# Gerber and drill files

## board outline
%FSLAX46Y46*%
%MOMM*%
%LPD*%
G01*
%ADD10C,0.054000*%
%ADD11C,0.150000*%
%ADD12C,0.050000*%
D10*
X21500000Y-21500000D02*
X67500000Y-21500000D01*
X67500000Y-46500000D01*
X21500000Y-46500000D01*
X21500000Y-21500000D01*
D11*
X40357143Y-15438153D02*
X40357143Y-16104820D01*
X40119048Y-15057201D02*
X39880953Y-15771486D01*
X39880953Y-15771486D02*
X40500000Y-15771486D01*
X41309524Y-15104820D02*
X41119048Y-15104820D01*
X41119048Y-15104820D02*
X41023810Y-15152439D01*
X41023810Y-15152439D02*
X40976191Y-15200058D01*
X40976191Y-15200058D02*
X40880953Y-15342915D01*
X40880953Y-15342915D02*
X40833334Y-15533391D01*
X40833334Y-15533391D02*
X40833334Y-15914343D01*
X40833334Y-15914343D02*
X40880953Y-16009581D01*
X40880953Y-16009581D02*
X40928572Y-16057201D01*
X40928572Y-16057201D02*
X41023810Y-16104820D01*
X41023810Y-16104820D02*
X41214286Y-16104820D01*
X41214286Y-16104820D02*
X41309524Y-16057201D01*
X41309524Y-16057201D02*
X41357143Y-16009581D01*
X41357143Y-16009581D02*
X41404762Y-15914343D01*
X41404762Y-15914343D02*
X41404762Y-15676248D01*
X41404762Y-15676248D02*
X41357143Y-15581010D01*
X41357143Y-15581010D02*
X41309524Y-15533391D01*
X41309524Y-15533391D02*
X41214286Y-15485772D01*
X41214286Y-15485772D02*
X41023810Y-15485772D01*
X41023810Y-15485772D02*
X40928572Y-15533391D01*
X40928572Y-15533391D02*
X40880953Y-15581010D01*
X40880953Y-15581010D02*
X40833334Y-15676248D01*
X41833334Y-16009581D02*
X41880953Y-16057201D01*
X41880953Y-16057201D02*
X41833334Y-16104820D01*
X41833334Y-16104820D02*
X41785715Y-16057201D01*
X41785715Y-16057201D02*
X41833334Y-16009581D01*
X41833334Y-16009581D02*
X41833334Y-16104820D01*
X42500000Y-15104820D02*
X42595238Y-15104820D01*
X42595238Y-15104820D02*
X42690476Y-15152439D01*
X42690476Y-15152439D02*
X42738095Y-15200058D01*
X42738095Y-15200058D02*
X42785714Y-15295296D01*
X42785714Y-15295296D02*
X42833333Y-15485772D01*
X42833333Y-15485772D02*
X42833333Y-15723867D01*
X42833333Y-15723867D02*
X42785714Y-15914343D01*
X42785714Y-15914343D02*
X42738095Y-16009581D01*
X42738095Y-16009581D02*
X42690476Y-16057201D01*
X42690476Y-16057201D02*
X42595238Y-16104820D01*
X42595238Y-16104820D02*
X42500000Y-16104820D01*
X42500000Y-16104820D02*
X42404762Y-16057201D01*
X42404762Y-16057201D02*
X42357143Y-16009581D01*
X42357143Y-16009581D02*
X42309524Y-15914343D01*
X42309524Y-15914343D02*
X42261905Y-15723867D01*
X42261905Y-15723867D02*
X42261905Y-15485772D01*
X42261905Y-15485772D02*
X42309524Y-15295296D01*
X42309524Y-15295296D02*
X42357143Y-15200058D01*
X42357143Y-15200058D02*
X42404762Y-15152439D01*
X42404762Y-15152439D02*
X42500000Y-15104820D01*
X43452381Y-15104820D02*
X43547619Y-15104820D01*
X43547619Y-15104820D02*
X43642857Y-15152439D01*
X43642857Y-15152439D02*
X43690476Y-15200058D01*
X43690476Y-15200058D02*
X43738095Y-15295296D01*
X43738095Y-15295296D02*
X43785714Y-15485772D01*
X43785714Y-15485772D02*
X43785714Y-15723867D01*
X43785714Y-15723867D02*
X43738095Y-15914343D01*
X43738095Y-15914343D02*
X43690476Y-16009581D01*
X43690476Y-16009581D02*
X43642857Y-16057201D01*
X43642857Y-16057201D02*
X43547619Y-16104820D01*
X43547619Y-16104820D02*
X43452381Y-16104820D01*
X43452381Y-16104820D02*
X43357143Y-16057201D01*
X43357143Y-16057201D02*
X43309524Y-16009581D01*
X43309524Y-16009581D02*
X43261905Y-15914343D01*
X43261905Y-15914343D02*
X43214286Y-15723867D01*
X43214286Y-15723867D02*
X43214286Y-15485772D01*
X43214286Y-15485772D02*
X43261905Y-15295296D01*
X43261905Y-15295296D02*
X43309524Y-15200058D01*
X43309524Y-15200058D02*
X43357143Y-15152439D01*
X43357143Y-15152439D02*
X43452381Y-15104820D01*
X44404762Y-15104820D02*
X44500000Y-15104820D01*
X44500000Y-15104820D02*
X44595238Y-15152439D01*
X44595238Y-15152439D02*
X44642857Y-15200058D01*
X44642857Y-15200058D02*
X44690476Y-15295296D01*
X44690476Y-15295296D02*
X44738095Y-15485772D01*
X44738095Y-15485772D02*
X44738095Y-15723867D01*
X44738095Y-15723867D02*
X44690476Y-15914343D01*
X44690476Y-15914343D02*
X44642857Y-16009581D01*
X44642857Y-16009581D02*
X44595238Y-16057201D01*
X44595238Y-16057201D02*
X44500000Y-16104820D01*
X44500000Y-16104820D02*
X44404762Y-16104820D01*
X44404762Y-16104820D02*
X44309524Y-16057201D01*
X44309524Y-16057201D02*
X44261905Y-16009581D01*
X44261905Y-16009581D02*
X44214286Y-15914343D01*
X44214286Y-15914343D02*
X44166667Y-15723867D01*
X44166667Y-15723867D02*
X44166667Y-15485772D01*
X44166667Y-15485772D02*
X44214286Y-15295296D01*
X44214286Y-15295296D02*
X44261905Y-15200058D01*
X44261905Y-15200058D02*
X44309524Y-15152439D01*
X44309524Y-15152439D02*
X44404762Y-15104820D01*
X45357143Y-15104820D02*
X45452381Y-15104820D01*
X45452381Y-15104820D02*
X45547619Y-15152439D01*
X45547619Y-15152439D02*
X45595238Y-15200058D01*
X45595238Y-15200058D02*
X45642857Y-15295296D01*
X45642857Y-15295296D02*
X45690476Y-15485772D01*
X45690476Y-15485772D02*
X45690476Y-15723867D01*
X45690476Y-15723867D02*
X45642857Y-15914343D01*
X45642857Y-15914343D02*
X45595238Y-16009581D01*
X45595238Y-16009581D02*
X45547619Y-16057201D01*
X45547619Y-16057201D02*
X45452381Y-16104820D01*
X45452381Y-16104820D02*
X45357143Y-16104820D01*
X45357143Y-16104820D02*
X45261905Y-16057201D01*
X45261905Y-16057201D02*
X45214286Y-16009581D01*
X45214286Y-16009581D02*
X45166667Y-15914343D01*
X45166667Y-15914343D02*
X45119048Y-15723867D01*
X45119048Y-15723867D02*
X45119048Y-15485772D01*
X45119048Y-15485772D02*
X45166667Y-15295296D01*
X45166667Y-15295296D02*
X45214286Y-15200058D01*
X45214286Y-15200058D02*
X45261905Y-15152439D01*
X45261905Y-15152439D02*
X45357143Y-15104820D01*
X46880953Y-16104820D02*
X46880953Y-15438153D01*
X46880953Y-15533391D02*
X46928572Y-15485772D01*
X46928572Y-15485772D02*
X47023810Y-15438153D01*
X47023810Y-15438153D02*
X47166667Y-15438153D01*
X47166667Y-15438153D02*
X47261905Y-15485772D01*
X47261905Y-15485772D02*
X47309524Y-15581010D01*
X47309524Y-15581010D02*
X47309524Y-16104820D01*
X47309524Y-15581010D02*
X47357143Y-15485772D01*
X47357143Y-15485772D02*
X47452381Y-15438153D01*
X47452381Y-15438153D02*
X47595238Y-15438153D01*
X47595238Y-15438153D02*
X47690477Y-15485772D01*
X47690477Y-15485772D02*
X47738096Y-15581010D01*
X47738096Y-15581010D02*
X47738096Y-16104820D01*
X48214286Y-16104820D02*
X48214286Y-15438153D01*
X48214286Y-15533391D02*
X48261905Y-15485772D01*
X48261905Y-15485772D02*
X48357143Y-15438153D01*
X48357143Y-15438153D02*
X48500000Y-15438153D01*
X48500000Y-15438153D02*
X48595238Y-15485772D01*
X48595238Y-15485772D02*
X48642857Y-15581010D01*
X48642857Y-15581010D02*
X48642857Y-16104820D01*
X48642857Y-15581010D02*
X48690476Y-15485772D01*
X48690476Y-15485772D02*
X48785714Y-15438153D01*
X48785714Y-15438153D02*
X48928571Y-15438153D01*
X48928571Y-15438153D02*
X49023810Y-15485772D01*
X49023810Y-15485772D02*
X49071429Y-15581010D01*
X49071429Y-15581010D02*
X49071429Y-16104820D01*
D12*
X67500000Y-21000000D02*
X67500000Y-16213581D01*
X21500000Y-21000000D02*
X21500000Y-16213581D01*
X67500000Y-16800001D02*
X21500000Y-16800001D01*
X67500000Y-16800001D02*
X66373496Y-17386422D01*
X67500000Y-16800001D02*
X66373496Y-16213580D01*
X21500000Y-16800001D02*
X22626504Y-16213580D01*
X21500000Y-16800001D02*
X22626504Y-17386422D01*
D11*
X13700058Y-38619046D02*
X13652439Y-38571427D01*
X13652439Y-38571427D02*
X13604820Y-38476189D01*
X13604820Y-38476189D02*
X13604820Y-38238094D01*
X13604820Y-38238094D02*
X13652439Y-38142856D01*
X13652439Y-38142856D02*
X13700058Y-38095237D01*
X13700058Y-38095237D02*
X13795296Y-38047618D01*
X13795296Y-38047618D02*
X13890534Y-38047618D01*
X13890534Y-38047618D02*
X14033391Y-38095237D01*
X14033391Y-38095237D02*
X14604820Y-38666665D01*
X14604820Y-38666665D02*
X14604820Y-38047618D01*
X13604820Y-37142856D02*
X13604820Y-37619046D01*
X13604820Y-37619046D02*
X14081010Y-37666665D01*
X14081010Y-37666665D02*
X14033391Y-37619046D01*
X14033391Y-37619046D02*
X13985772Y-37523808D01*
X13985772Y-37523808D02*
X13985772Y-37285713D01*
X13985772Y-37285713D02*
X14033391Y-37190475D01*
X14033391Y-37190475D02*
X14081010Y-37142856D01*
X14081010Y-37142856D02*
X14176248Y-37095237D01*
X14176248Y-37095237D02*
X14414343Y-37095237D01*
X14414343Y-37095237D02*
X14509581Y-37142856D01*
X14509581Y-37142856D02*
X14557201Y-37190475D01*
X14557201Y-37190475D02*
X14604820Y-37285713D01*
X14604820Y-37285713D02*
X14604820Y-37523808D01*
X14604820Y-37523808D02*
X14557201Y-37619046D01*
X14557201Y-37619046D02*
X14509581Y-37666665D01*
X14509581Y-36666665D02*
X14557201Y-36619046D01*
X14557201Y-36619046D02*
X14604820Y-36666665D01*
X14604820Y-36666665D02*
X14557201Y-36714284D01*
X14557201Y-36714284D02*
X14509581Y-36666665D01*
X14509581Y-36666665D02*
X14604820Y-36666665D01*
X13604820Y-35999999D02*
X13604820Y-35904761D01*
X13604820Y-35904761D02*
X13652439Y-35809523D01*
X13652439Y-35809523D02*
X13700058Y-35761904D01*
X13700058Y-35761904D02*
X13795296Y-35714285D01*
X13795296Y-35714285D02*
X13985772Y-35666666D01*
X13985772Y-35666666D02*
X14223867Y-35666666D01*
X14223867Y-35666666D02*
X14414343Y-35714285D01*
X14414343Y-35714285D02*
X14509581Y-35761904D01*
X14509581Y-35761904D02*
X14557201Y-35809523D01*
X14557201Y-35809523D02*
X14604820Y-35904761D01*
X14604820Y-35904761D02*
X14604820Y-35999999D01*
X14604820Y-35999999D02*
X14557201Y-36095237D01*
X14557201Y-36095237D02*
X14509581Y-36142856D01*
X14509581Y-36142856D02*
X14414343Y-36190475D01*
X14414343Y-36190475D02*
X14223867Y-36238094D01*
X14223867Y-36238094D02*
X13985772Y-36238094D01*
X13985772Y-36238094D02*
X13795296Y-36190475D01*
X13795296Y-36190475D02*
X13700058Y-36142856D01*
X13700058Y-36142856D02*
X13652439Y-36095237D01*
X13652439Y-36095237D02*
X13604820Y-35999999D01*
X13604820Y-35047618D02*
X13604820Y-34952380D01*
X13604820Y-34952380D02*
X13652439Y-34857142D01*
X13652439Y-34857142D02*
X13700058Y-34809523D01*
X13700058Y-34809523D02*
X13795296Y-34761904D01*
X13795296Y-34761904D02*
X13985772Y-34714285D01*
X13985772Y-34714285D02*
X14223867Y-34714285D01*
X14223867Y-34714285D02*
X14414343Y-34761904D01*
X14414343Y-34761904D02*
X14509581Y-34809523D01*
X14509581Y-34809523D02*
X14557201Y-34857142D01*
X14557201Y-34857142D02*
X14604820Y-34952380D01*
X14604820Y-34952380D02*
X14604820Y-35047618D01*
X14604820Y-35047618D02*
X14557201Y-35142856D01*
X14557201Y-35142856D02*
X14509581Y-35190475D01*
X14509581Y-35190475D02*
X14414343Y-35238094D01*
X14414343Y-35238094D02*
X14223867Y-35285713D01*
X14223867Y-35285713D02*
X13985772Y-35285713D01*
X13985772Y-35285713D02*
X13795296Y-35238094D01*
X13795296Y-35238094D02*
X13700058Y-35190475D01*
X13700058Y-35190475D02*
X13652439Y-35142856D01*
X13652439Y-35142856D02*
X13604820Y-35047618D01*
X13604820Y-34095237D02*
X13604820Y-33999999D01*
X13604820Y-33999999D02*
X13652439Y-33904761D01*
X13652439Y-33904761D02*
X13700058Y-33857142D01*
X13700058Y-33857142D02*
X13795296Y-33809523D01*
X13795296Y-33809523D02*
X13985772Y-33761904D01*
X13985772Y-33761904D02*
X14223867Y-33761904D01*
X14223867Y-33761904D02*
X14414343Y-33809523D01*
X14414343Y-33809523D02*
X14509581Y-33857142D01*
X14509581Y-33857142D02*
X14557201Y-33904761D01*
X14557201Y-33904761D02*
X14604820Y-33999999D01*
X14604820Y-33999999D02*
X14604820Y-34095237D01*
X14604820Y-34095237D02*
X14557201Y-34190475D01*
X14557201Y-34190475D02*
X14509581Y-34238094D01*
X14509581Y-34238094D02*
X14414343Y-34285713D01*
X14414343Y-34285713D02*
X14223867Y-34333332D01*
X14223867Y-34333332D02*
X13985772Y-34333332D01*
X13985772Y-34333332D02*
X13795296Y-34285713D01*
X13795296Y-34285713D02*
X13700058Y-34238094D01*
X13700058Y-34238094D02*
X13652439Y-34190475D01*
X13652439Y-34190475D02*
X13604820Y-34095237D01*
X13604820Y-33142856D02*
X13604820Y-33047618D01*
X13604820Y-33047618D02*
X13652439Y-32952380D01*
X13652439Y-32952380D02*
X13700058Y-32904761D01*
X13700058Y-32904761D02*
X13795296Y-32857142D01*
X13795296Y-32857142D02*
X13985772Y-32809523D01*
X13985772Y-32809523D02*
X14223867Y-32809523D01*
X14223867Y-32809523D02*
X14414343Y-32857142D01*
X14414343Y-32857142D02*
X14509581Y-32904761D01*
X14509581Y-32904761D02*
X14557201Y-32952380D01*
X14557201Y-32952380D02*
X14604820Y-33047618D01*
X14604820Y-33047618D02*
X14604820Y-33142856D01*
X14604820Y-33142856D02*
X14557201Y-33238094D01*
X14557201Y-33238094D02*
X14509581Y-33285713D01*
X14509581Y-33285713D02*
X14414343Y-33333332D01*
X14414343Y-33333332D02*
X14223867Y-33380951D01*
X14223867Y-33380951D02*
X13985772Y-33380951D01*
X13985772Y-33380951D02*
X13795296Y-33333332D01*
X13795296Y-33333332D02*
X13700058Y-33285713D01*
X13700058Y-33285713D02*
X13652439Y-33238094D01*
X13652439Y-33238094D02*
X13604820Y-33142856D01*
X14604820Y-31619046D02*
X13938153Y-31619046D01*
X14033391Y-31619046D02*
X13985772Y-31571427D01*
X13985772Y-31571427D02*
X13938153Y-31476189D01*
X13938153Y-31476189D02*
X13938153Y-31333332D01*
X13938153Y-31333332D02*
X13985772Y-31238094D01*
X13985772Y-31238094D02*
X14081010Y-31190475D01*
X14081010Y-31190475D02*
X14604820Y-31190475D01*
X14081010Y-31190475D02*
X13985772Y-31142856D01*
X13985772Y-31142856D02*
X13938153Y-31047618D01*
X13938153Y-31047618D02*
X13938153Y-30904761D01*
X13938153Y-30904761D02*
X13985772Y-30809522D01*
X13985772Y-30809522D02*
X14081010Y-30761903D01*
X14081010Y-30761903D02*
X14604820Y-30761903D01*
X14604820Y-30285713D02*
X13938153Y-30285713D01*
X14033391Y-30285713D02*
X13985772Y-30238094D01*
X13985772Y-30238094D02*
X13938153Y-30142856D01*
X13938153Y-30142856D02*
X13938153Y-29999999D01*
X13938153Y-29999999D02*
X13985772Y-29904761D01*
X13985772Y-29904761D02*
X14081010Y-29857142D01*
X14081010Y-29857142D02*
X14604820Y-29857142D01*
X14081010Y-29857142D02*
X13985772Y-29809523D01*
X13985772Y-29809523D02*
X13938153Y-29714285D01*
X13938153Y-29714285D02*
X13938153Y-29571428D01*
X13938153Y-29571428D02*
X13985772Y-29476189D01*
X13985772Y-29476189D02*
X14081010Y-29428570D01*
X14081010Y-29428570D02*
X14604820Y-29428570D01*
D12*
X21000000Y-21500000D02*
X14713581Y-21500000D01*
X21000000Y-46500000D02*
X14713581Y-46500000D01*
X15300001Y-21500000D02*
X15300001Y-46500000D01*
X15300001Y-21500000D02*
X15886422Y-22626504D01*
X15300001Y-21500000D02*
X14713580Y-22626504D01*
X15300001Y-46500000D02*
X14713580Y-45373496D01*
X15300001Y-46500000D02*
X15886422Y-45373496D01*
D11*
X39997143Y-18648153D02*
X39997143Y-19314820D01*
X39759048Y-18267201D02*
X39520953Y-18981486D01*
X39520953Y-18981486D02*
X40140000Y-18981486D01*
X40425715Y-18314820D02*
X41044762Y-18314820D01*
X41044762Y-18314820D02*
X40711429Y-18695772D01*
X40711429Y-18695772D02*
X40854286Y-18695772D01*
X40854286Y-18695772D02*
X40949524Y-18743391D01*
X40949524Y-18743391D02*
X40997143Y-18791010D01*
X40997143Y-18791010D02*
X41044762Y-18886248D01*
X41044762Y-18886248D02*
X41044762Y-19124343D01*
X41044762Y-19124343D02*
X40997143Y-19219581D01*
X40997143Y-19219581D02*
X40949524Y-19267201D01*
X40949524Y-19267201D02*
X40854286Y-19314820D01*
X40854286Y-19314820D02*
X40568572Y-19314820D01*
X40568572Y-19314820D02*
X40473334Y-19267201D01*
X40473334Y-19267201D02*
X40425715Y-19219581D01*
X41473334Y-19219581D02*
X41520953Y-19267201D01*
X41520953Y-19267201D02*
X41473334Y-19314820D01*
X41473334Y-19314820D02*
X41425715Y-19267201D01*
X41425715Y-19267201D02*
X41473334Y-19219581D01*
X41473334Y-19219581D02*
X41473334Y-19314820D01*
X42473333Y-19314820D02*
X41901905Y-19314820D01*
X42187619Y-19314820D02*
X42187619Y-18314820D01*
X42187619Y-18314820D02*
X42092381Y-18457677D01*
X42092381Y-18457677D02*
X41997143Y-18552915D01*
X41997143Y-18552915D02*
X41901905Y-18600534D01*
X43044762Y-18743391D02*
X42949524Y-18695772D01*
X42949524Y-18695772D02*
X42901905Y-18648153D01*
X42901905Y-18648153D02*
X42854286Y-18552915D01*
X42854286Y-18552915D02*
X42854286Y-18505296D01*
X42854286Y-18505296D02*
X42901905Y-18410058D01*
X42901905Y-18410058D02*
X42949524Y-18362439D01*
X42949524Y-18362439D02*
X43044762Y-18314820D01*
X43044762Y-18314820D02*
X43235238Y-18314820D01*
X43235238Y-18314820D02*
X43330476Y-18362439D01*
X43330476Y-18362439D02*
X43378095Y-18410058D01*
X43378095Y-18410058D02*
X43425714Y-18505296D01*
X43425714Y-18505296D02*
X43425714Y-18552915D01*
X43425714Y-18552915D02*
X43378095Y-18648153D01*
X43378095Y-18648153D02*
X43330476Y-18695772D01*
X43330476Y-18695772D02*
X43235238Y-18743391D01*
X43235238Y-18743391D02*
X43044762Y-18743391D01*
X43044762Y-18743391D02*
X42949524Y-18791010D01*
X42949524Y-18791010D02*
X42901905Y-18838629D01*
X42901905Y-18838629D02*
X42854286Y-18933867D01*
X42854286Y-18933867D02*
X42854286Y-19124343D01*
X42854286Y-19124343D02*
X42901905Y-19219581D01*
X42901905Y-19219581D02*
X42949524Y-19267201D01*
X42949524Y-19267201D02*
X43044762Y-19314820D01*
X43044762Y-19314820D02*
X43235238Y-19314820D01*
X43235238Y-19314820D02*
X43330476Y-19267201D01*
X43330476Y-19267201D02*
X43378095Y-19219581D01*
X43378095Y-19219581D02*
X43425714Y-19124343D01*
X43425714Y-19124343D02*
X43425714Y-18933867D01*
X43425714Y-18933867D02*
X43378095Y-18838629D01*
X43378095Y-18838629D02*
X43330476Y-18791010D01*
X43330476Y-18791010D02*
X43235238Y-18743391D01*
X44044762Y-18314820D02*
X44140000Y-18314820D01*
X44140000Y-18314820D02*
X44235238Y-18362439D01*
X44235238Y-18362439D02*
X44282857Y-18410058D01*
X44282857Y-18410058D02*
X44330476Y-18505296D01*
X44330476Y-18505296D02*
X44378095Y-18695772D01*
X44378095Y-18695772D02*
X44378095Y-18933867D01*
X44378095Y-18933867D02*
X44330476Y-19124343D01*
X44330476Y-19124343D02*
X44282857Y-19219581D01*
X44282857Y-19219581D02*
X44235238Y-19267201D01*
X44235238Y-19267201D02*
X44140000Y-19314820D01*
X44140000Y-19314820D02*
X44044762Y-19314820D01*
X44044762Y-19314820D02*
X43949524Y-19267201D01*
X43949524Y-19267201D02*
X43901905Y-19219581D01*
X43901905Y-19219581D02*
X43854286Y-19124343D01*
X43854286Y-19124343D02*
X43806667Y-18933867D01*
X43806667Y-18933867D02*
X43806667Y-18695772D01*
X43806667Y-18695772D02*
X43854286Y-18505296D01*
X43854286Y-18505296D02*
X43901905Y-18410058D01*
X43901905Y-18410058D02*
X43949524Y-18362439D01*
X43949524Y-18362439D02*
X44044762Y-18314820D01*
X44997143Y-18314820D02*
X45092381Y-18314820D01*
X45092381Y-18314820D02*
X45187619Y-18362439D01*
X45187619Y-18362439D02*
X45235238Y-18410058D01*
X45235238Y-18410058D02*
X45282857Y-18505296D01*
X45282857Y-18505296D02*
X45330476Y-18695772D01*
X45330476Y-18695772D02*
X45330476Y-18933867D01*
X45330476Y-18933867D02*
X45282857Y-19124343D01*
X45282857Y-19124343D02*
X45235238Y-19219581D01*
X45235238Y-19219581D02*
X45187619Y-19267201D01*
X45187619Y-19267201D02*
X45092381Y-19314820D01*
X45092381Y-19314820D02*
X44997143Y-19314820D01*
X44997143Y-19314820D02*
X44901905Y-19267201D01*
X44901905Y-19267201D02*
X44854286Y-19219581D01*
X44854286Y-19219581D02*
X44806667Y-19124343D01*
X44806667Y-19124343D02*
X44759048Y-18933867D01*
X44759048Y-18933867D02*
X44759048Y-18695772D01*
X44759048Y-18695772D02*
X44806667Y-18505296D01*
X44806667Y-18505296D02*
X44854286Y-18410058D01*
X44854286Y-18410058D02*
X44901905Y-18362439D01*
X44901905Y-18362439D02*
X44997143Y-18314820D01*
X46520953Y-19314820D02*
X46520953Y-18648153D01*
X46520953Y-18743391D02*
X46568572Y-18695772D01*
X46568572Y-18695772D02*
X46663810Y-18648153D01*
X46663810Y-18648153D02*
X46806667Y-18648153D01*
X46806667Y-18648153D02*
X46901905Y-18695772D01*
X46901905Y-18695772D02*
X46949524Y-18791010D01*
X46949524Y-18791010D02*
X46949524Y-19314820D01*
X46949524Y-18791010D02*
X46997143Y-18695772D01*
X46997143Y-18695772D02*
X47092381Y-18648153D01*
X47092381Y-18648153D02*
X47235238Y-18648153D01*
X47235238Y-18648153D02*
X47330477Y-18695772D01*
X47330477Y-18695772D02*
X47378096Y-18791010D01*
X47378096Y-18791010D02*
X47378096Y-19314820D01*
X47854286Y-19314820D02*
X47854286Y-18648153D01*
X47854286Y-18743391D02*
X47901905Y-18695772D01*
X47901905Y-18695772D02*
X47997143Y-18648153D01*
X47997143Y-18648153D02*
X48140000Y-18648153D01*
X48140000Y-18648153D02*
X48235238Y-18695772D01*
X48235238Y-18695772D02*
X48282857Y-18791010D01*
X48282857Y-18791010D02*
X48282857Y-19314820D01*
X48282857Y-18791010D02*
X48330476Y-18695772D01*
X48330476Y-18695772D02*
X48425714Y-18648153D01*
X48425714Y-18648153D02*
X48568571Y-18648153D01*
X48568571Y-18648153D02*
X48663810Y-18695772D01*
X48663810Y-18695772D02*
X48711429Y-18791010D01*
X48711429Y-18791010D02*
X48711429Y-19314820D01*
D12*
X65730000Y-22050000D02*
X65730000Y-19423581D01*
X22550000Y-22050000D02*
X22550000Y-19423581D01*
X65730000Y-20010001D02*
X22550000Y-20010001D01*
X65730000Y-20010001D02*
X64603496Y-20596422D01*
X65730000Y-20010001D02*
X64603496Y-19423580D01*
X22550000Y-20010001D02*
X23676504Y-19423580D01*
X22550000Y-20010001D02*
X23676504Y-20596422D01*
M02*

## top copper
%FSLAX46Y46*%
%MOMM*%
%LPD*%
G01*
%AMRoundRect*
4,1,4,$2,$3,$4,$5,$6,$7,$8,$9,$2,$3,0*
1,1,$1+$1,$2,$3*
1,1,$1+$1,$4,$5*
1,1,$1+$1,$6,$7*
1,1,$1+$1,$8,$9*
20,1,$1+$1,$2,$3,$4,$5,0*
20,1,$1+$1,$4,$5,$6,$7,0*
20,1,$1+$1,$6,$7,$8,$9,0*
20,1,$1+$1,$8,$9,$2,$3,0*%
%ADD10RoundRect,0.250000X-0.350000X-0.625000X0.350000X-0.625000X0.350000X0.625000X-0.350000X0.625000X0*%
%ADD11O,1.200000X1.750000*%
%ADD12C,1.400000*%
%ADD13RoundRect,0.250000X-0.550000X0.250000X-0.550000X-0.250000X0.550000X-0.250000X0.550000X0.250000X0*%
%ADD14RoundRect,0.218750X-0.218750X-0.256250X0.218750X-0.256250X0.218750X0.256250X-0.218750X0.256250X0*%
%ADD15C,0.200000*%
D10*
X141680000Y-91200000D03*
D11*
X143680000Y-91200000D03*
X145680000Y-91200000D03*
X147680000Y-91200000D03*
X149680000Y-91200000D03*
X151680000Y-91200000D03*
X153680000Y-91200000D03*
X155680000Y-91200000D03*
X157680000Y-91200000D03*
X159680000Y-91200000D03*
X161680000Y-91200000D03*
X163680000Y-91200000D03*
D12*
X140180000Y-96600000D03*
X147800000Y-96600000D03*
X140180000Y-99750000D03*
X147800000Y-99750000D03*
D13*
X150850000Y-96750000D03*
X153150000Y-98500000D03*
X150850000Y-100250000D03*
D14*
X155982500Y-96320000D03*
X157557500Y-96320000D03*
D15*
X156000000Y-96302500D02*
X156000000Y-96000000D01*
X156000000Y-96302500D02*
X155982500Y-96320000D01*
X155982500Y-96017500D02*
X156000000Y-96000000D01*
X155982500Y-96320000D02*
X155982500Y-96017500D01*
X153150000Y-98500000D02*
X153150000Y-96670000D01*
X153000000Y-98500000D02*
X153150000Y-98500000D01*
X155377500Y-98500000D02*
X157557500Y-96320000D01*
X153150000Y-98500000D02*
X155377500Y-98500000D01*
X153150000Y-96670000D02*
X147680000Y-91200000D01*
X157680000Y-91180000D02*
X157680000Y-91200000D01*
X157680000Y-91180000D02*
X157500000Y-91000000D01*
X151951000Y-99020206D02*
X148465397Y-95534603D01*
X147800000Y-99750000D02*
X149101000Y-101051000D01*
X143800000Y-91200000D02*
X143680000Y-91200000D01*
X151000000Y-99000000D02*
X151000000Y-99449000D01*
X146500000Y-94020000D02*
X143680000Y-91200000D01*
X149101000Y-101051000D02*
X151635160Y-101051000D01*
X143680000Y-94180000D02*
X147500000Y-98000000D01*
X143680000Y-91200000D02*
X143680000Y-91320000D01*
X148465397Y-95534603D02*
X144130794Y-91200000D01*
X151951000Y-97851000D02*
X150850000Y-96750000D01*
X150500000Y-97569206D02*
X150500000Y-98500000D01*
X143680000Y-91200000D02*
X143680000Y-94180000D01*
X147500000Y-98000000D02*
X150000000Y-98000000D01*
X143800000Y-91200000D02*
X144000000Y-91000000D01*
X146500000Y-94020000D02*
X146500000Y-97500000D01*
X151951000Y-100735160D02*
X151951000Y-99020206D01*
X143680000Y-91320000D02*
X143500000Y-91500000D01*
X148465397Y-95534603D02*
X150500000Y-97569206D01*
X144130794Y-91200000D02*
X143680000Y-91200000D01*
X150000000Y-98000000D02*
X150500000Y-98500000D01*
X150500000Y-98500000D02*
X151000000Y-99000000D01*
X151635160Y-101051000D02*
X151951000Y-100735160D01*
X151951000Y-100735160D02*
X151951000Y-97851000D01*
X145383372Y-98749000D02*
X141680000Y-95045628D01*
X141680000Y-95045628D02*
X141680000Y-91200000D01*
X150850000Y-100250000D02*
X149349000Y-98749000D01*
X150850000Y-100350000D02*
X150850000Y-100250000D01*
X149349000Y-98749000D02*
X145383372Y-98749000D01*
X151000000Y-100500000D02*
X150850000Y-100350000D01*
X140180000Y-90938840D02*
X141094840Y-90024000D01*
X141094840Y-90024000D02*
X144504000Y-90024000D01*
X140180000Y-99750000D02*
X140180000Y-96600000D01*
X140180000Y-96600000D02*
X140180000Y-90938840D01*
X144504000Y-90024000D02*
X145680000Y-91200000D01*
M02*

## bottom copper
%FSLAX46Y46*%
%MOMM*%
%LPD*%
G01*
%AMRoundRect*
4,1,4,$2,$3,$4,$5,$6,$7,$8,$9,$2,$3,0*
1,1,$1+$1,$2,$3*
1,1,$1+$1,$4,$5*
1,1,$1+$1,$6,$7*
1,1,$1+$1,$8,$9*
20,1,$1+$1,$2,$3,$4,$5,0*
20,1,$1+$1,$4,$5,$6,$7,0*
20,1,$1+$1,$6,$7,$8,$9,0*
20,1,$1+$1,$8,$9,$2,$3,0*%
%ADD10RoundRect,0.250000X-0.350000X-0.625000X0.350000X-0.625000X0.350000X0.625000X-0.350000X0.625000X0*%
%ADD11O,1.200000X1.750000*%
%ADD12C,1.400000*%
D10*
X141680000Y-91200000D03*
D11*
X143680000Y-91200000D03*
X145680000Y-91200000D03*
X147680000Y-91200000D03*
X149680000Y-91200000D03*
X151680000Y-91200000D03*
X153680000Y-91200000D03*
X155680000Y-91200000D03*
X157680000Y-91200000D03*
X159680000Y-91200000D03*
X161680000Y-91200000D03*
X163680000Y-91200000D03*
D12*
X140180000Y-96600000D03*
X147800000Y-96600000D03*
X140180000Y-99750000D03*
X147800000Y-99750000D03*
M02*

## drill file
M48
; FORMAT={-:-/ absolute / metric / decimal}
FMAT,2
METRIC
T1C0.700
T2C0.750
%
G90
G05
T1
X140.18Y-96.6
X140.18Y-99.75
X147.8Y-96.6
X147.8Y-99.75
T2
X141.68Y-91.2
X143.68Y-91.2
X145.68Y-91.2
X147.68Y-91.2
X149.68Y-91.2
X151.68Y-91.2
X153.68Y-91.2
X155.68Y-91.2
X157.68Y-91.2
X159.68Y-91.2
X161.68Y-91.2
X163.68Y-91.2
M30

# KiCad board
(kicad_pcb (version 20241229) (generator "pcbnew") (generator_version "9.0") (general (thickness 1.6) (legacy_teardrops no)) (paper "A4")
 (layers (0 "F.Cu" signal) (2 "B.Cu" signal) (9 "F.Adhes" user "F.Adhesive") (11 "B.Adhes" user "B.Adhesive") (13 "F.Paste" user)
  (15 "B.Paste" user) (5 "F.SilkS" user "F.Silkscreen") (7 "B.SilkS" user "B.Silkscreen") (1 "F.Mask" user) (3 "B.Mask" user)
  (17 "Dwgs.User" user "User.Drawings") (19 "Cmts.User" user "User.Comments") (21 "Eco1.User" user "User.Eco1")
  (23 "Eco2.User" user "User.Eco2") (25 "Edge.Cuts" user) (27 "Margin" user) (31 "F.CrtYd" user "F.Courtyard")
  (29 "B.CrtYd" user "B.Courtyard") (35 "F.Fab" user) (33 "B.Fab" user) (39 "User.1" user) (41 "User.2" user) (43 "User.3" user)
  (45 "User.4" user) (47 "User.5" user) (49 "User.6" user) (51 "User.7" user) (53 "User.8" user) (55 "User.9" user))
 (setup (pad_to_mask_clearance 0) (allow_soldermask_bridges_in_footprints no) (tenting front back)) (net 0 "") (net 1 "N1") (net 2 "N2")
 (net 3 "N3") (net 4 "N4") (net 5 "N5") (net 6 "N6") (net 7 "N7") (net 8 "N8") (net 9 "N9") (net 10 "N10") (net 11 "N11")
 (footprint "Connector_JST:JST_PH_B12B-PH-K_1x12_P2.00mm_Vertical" (layer "F.Cu") (at 141.68 91.2)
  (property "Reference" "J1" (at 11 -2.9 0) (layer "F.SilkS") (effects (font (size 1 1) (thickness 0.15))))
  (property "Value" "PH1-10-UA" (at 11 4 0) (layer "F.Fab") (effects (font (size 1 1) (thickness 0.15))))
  (pad "1" thru_hole roundrect (at 0 0) (size 1.2 1.75) (drill 0.75) (layers "*.Cu" "*.Mask") (remove_unused_layers no)
   (roundrect_rratio 0.208333) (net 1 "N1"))
  (pad "2" thru_hole oval (at 2 0) (size 1.2 1.75) (drill 0.75) (layers "*.Cu" "*.Mask") (remove_unused_layers no) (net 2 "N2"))
  (pad "3" thru_hole oval (at 4 0) (size 1.2 1.75) (drill 0.75) (layers "*.Cu" "*.Mask") (remove_unused_layers no) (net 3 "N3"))
  (pad "4" thru_hole oval (at 6 0) (size 1.2 1.75) (drill 0.75) (layers "*.Cu" "*.Mask") (remove_unused_layers no) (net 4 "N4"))
  (pad "5" thru_hole oval (at 8 0) (size 1.2 1.75) (drill 0.75) (layers "*.Cu" "*.Mask") (remove_unused_layers no) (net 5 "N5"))
  (pad "6" thru_hole oval (at 10 0) (size 1.2 1.75) (drill 0.75) (layers "*.Cu" "*.Mask") (remove_unused_layers no) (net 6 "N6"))
  (pad "7" thru_hole oval (at 12 0) (size 1.2 1.75) (drill 0.75) (layers "*.Cu" "*.Mask") (remove_unused_layers no) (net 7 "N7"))
  (pad "8" thru_hole oval (at 14 0) (size 1.2 1.75) (drill 0.75) (layers "*.Cu" "*.Mask") (remove_unused_layers no) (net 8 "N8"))
  (pad "9" thru_hole oval (at 16 0) (size 1.2 1.75) (drill 0.75) (layers "*.Cu" "*.Mask") (remove_unused_layers no) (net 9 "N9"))
  (pad "10" thru_hole oval (at 18 0) (size 1.2 1.75) (drill 0.75) (layers "*.Cu" "*.Mask") (remove_unused_layers no) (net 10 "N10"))
  (pad "11" thru_hole oval (at 20 0) (size 1.2 1.75) (drill 0.75) (layers "*.Cu" "*.Mask") (remove_unused_layers no))
  (pad "12" thru_hole oval (at 22 0) (size 1.2 1.75) (drill 0.75) (layers "*.Cu" "*.Mask") (remove_unused_layers no)))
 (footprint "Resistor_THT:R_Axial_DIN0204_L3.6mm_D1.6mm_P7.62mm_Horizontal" (layer "F.Cu") (at 140.18 96.6)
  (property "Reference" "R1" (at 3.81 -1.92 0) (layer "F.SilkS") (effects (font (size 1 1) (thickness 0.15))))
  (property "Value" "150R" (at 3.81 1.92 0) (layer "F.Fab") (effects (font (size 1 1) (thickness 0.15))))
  (pad "1" thru_hole circle (at 0 0) (size 1.4 1.4) (drill 0.7) (layers "*.Cu" "*.Mask") (remove_unused_layers no) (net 3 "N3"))
  (pad "2" thru_hole circle (at 7.62 0) (size 1.4 1.4) (drill 0.7) (layers "*.Cu" "*.Mask") (remove_unused_layers no) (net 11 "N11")))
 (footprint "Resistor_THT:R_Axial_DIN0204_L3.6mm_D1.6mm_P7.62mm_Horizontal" (layer "F.Cu") (at 140.18 99.75)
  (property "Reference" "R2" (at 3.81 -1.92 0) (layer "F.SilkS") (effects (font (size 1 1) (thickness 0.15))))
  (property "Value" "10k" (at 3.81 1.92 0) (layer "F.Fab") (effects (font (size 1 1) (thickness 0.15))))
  (pad "1" thru_hole circle (at 0 0) (size 1.4 1.4) (drill 0.7) (layers "*.Cu" "*.Mask") (remove_unused_layers no) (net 3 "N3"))
  (pad "2" thru_hole circle (at 7.62 0) (size 1.4 1.4) (drill 0.7) (layers "*.Cu" "*.Mask") (remove_unused_layers no) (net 2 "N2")))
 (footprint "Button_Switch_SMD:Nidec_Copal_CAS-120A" (layer "F.Cu") (at 152 98.5)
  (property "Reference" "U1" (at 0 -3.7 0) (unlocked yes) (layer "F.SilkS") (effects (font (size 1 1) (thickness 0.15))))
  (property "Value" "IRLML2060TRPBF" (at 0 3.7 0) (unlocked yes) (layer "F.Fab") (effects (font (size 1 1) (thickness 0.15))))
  (pad "1" smd roundrect (at -1.15 -1.75 270) (size 1 1.6) (layers "F.Cu" "F.Mask" "F.Paste") (roundrect_rratio 0.25) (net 2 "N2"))
  (pad "2" smd roundrect (at 1.15 0 270) (size 1 1.6) (layers "F.Cu" "F.Mask" "F.Paste") (roundrect_rratio 0.25) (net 4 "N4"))
  (pad "3" smd roundrect (at -1.15 1.75 270) (size 1 1.6) (layers "F.Cu" "F.Mask" "F.Paste") (roundrect_rratio 0.25) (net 1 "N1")))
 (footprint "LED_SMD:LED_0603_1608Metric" (layer "F.Cu") (at 156.77 96.32)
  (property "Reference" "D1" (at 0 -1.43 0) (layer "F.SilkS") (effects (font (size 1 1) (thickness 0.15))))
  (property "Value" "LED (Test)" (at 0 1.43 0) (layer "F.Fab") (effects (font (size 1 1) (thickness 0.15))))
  (pad "1" smd roundrect (at -0.7875 0) (size 0.875 0.95) (layers "F.Cu" "F.Mask" "F.Paste") (roundrect_rratio 0.25) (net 11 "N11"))
  (pad "2" smd roundrect (at 0.7875 0) (size 0.875 0.95) (layers "F.Cu" "F.Mask" "F.Paste") (roundrect_rratio 0.25) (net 4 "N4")))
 (gr_rect (start 21.5 21.5) (end 67.5 46.5) (stroke (width 0.054) (type default)) (fill no) (layer "Edge.Cuts"))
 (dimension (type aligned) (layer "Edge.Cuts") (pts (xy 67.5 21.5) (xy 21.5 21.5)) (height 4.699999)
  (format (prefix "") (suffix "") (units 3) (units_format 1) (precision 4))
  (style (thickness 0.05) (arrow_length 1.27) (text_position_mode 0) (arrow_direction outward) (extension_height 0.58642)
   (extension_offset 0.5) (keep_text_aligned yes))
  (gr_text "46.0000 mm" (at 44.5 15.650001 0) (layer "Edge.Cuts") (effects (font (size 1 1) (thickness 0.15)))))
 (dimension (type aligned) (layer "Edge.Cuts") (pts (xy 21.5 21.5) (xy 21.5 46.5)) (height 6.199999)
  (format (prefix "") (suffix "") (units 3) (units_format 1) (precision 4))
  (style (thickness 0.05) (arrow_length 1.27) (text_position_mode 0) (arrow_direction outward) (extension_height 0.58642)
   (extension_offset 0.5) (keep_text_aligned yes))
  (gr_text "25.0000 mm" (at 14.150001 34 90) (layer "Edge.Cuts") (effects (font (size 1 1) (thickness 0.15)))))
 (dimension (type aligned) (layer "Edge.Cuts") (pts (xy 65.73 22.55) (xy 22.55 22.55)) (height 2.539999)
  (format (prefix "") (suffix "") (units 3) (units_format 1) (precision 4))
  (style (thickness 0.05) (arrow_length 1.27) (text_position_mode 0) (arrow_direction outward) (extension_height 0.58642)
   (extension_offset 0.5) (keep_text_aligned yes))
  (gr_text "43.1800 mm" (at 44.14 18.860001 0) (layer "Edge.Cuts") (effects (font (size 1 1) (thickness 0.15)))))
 (segment (start 156 96.3025) (end 156 96) (width 0.2) (layer "F.Cu") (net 11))
 (segment (start 156 96.3025) (end 155.9825 96.32) (width 0.2) (layer "F.Cu") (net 11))
 (segment (start 155.9825 96.0175) (end 156 96) (width 0.2) (layer "F.Cu") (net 11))
 (segment (start 155.9825 96.32) (end 155.9825 96.0175) (width 0.2) (layer "F.Cu") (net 11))
 (segment (start 153.15 98.5) (end 153.15 96.67) (width 0.2) (layer "F.Cu") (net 4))
 (segment (start 153 98.5) (end 153.15 98.5) (width 0.2) (layer "F.Cu") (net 4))
 (segment (start 155.3775 98.5) (end 157.5575 96.32) (width 0.2) (layer "F.Cu") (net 4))
 (segment (start 153.15 98.5) (end 155.3775 98.5) (width 0.2) (layer "F.Cu") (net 4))
 (segment (start 153.15 96.67) (end 147.68 91.2) (width 0.2) (layer "F.Cu") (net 4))
 (segment (start 157.68 91.18) (end 157.68 91.2) (width 0.2) (layer "F.Cu") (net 9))
 (segment (start 157.68 91.18) (end 157.5 91) (width 0.2) (layer "F.Cu") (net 9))
 (segment (start 151.951 99.020206) (end 148.465397 95.534603) (width 0.2) (layer "F.Cu") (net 2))
 (segment (start 147.8 99.75) (end 149.101 101.051) (width 0.2) (layer "F.Cu") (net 2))
 (segment (start 143.8 91.2) (end 143.68 91.2) (width 0.2) (layer "F.Cu") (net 2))
 (segment (start 151 99) (end 151 99.449) (width 0.2) (layer "F.Cu") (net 2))
 (segment (start 146.5 94.02) (end 143.68 91.2) (width 0.2) (layer "F.Cu") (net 2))
 (segment (start 149.101 101.051) (end 151.63516 101.051) (width 0.2) (layer "F.Cu") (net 2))
 (segment (start 143.68 94.18) (end 147.5 98) (width 0.2) (layer "F.Cu") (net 2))
 (segment (start 143.68 91.2) (end 143.68 91.32) (width 0.2) (layer "F.Cu") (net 2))
 (segment (start 148.465397 95.534603) (end 144.130794 91.2) (width 0.2) (layer "F.Cu") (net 2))
 (segment (start 151.951 97.851) (end 150.85 96.75) (width 0.2) (layer "F.Cu") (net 2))
 (segment (start 150.5 97.569206) (end 150.5 98.5) (width 0.2) (layer "F.Cu") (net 2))
 (segment (start 143.68 91.2) (end 143.68 94.18) (width 0.2) (layer "F.Cu") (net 2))
 (segment (start 147.5 98) (end 150 98) (width 0.2) (layer "F.Cu") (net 2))
 (segment (start 143.8 91.2) (end 144 91) (width 0.2) (layer "F.Cu") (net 2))
 (segment (start 146.5 94.02) (end 146.5 97.5) (width 0.2) (layer "F.Cu") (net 2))
 (segment (start 151.951 100.73516) (end 151.951 99.020206) (width 0.2) (layer "F.Cu") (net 2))
 (segment (start 143.68 91.32) (end 143.5 91.5) (width 0.2) (layer "F.Cu") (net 2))
 (segment (start 148.465397 95.534603) (end 150.5 97.569206) (width 0.2) (layer "F.Cu") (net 2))
 (segment (start 144.130794 91.2) (end 143.68 91.2) (width 0.2) (layer "F.Cu") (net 2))
 (segment (start 150 98) (end 150.5 98.5) (width 0.2) (layer "F.Cu") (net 2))
 (segment (start 150.5 98.5) (end 151 99) (width 0.2) (layer "F.Cu") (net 2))
 (segment (start 151.63516 101.051) (end 151.951 100.73516) (width 0.2) (layer "F.Cu") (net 2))
 (segment (start 151.951 100.73516) (end 151.951 97.851) (width 0.2) (layer "F.Cu") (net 2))
 (segment (start 145.383372 98.749) (end 141.68 95.045628) (width 0.2) (layer "F.Cu") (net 1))
 (segment (start 141.68 95.045628) (end 141.68 91.2) (width 0.2) (layer "F.Cu") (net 1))
 (segment (start 150.85 100.25) (end 149.349 98.749) (width 0.2) (layer "F.Cu") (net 1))
 (segment (start 150.85 100.35) (end 150.85 100.25) (width 0.2) (layer "F.Cu") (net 1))
 (segment (start 149.349 98.749) (end 145.383372 98.749) (width 0.2) (layer "F.Cu") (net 1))
 (segment (start 151 100.5) (end 150.85 100.35) (width 0.2) (layer "F.Cu") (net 1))
 (segment (start 140.18 90.93884) (end 141.09484 90.024) (width 0.2) (layer "F.Cu") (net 3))
 (segment (start 141.09484 90.024) (end 144.504 90.024) (width 0.2) (layer "F.Cu") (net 3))
 (segment (start 140.18 99.75) (end 140.18 96.6) (width 0.2) (layer "F.Cu") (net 3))
 (segment (start 140.18 96.6) (end 140.18 90.93884) (width 0.2) (layer "F.Cu") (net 3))
 (segment (start 144.504 90.024) (end 145.68 91.2) (width 0.2) (layer "F.Cu") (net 3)))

